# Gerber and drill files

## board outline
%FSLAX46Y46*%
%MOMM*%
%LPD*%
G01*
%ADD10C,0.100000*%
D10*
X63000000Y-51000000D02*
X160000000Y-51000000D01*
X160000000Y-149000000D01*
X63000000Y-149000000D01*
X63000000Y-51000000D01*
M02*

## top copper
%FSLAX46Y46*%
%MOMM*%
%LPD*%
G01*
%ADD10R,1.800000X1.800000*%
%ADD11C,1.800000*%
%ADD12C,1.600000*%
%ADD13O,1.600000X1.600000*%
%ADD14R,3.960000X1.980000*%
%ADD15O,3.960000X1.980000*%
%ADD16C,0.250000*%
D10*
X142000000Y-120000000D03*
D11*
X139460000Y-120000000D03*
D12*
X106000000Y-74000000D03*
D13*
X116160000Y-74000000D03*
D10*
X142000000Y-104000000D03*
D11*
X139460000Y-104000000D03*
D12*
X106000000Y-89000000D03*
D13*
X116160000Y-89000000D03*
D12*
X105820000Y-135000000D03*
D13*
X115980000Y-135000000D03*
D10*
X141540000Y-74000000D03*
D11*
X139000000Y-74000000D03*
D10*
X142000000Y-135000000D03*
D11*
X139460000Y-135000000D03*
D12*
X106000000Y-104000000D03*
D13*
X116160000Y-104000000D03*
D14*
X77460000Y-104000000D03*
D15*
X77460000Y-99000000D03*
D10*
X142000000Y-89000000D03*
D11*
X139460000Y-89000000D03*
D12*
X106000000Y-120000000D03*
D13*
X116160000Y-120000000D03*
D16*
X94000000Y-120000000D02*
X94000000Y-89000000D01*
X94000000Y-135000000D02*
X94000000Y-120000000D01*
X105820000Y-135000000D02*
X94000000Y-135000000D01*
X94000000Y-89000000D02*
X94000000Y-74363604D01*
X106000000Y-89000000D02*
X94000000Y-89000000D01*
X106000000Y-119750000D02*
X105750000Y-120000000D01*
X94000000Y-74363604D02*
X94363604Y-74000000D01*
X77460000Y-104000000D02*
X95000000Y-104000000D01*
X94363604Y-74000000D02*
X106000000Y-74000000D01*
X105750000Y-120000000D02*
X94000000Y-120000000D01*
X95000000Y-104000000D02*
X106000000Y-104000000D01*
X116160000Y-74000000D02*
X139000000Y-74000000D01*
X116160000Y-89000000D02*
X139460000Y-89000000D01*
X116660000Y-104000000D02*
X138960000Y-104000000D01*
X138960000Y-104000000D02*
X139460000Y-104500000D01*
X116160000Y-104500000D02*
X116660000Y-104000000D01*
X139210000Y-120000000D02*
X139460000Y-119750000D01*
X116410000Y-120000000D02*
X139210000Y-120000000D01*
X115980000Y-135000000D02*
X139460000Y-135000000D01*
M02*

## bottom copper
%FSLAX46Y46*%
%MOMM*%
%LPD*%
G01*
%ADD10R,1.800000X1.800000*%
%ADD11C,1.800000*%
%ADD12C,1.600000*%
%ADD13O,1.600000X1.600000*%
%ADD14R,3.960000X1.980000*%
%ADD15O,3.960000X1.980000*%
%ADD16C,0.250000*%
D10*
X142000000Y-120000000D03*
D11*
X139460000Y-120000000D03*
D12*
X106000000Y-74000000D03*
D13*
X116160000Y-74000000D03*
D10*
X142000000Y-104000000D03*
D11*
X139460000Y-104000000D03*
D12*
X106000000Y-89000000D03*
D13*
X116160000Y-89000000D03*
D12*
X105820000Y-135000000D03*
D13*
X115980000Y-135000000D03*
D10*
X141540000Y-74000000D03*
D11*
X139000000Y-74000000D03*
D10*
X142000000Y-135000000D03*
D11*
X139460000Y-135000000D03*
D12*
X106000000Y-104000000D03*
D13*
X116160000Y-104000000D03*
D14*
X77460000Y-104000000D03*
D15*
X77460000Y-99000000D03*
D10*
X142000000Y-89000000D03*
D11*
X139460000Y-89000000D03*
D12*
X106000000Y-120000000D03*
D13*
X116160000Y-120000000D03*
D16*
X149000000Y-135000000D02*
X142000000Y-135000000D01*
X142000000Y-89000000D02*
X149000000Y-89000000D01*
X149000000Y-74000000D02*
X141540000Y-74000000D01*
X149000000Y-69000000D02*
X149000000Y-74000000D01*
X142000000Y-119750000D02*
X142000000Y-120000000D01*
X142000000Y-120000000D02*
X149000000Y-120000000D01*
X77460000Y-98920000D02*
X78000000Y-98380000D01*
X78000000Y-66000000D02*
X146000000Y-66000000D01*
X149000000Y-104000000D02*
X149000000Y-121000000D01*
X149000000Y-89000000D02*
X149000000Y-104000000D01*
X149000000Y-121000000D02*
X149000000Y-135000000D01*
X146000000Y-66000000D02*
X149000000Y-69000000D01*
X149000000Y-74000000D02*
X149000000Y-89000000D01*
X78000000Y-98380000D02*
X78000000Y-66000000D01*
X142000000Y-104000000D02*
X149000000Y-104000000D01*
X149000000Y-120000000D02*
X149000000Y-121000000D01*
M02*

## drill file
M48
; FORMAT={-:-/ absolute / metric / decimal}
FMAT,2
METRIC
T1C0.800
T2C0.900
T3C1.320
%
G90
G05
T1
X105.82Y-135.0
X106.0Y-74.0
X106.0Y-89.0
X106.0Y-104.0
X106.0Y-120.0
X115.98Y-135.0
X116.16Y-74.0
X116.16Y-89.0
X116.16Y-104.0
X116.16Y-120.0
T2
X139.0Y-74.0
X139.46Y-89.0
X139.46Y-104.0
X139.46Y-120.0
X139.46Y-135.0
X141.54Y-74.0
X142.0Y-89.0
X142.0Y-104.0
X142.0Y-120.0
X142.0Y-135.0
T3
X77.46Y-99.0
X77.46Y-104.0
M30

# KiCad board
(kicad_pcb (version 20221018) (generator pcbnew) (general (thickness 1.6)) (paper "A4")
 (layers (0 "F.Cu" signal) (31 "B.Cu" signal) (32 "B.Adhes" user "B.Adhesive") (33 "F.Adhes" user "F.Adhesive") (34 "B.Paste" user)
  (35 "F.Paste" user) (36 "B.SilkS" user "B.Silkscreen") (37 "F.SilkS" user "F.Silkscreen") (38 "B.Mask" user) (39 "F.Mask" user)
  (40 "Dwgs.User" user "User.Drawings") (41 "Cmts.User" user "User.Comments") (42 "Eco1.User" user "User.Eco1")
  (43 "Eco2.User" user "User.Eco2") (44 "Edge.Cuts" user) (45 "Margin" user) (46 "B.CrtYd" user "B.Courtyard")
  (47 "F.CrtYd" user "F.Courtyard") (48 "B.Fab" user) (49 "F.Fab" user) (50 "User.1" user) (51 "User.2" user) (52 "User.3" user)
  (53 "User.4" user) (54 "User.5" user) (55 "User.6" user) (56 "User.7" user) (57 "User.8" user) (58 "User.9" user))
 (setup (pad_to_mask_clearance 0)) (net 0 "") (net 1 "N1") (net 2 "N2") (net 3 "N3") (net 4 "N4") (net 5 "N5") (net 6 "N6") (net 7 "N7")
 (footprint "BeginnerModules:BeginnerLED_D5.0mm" (layer "F.Cu") (at 142 120 180)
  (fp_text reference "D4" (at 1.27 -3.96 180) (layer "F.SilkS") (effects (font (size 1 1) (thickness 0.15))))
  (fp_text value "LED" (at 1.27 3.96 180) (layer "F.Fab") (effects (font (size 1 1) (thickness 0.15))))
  (pad "1" thru_hole rect (at 0 0 180) (size 1.8 1.8) (drill 0.9) (layers "*.Cu" "*.Mask") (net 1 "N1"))
  (pad "2" thru_hole circle (at 2.54 0 180) (size 1.8 1.8) (drill 0.9) (layers "*.Cu" "*.Mask") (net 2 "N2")))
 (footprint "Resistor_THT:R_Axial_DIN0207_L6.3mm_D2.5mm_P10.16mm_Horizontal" (layer "F.Cu") (at 106 74)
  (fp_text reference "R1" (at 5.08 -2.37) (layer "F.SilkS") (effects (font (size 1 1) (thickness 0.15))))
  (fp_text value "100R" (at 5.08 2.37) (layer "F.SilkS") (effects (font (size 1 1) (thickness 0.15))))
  (pad "1" thru_hole circle (at 0 0) (size 1.6 1.6) (drill 0.8) (layers "*.Cu" "*.Mask") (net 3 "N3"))
  (pad "2" thru_hole oval (at 10.16 0) (size 1.6 1.6) (drill 0.8) (layers "*.Cu" "*.Mask") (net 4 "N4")))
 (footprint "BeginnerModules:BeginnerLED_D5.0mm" (layer "F.Cu") (at 142 104 180)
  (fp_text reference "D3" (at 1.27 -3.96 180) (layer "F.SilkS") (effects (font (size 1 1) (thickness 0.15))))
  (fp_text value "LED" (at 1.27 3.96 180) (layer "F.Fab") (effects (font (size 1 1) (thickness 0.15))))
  (pad "1" thru_hole rect (at 0 0 180) (size 1.8 1.8) (drill 0.9) (layers "*.Cu" "*.Mask") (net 1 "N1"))
  (pad "2" thru_hole circle (at 2.54 0 180) (size 1.8 1.8) (drill 0.9) (layers "*.Cu" "*.Mask") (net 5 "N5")))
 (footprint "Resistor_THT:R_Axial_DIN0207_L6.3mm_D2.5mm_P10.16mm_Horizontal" (layer "F.Cu") (at 106 89)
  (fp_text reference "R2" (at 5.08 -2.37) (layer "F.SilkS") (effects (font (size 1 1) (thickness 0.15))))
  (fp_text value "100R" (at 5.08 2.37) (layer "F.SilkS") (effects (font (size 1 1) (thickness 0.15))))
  (pad "1" thru_hole circle (at 0 0) (size 1.6 1.6) (drill 0.8) (layers "*.Cu" "*.Mask") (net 3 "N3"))
  (pad "2" thru_hole oval (at 10.16 0) (size 1.6 1.6) (drill 0.8) (layers "*.Cu" "*.Mask") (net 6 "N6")))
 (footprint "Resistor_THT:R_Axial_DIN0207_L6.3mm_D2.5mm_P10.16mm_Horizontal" (layer "F.Cu") (at 105.82 135)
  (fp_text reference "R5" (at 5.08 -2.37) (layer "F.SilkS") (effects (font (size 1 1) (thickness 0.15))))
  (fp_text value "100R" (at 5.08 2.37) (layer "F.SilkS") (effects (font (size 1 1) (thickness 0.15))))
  (pad "1" thru_hole circle (at 0 0) (size 1.6 1.6) (drill 0.8) (layers "*.Cu" "*.Mask") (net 3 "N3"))
  (pad "2" thru_hole oval (at 10.16 0) (size 1.6 1.6) (drill 0.8) (layers "*.Cu" "*.Mask") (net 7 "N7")))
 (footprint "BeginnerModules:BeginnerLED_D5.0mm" (layer "F.Cu") (at 141.54 74 180)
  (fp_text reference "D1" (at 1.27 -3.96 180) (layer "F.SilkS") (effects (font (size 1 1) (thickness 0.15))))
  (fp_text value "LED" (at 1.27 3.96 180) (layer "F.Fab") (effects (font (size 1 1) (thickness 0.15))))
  (pad "1" thru_hole rect (at 0 0 180) (size 1.8 1.8) (drill 0.9) (layers "*.Cu" "*.Mask") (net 1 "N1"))
  (pad "2" thru_hole circle (at 2.54 0 180) (size 1.8 1.8) (drill 0.9) (layers "*.Cu" "*.Mask") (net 4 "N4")))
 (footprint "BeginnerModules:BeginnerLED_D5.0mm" (layer "F.Cu") (at 142 135 180)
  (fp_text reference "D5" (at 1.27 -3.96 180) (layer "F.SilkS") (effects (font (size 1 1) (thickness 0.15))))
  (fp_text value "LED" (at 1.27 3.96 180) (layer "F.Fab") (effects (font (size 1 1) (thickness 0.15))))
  (pad "1" thru_hole rect (at 0 0 180) (size 1.8 1.8) (drill 0.9) (layers "*.Cu" "*.Mask") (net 1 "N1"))
  (pad "2" thru_hole circle (at 2.54 0 180) (size 1.8 1.8) (drill 0.9) (layers "*.Cu" "*.Mask") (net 7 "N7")))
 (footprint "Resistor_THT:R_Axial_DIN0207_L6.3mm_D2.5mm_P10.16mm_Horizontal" (layer "F.Cu") (at 106 104)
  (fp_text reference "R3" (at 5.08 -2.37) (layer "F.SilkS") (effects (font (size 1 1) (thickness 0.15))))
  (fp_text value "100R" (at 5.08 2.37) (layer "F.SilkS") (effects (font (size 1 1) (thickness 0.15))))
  (pad "1" thru_hole circle (at 0 0) (size 1.6 1.6) (drill 0.8) (layers "*.Cu" "*.Mask") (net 3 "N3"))
  (pad "2" thru_hole oval (at 10.16 0) (size 1.6 1.6) (drill 0.8) (layers "*.Cu" "*.Mask") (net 5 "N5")))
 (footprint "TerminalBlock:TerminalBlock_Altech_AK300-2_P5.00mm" (layer "F.Cu") (at 77.46 104 90)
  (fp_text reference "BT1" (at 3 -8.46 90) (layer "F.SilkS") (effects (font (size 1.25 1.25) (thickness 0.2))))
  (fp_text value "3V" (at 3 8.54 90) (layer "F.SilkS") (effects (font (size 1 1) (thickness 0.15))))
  (pad "1" thru_hole rect (at 0 0 90) (size 1.98 3.96) (drill 1.32) (layers "*.Cu" "*.Mask") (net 3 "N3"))
  (pad "2" thru_hole oval (at 5 0 90) (size 1.98 3.96) (drill 1.32) (layers "*.Cu" "*.Mask") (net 1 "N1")))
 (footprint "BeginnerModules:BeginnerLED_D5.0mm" (layer "F.Cu") (at 142 89 180)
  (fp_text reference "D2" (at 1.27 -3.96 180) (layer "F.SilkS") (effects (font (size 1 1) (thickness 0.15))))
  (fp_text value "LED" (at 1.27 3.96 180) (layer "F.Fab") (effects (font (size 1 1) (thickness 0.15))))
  (pad "1" thru_hole rect (at 0 0 180) (size 1.8 1.8) (drill 0.9) (layers "*.Cu" "*.Mask") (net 1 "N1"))
  (pad "2" thru_hole circle (at 2.54 0 180) (size 1.8 1.8) (drill 0.9) (layers "*.Cu" "*.Mask") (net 6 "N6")))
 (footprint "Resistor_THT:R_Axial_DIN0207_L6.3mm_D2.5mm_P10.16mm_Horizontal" (layer "F.Cu") (at 106 120)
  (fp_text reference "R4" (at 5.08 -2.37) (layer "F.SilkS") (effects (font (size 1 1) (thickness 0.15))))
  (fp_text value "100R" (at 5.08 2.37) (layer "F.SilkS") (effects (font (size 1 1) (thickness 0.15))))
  (pad "1" thru_hole circle (at 0 0) (size 1.6 1.6) (drill 0.8) (layers "*.Cu" "*.Mask") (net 3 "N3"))
  (pad "2" thru_hole oval (at 10.16 0) (size 1.6 1.6) (drill 0.8) (layers "*.Cu" "*.Mask") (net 2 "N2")))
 (gr_rect (start 63 51) (end 160 149) (stroke (width 0.1) (type default)) (fill none) (layer "Edge.Cuts"))
 (segment (start 94 120) (end 94 89) (width 0.25) (layer "F.Cu") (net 3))
 (segment (start 94 135) (end 94 120) (width 0.25) (layer "F.Cu") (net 3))
 (segment (start 105.82 135) (end 94 135) (width 0.25) (layer "F.Cu") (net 3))
 (segment (start 94 89) (end 94 74.363604) (width 0.25) (layer "F.Cu") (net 3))
 (segment (start 106 89) (end 94 89) (width 0.25) (layer "F.Cu") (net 3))
 (segment (start 106 119.75) (end 105.75 120) (width 0.25) (layer "F.Cu") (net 3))
 (segment (start 94 74.363604) (end 94.363604 74) (width 0.25) (layer "F.Cu") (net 3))
 (segment (start 77.46 104) (end 95 104) (width 0.25) (layer "F.Cu") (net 3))
 (segment (start 94.363604 74) (end 106 74) (width 0.25) (layer "F.Cu") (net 3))
 (segment (start 105.75 120) (end 94 120) (width 0.25) (layer "F.Cu") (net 3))
 (segment (start 95 104) (end 106 104) (width 0.25) (layer "F.Cu") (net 3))
 (segment (start 149 135) (end 142 135) (width 0.25) (layer "B.Cu") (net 1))
 (segment (start 142 89) (end 149 89) (width 0.25) (layer "B.Cu") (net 1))
 (segment (start 149 74) (end 141.54 74) (width 0.25) (layer "B.Cu") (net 1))
 (segment (start 149 69) (end 149 74) (width 0.25) (layer "B.Cu") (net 1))
 (segment (start 142 119.75) (end 142 120) (width 0.25) (layer "B.Cu") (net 1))
 (segment (start 142 120) (end 149 120) (width 0.25) (layer "B.Cu") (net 1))
 (segment (start 77.46 98.92) (end 78 98.38) (width 0.25) (layer "B.Cu") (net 1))
 (segment (start 78 66) (end 146 66) (width 0.25) (layer "B.Cu") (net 1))
 (segment (start 149 104) (end 149 121) (width 0.25) (layer "B.Cu") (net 1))
 (segment (start 149 89) (end 149 104) (width 0.25) (layer "B.Cu") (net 1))
 (segment (start 149 121) (end 149 135) (width 0.25) (layer "B.Cu") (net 1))
 (segment (start 146 66) (end 149 69) (width 0.25) (layer "B.Cu") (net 1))
 (segment (start 149 74) (end 149 89) (width 0.25) (layer "B.Cu") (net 1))
 (segment (start 78 98.38) (end 78 66) (width 0.25) (layer "B.Cu") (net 1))
 (segment (start 142 104) (end 149 104) (width 0.25) (layer "B.Cu") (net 1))
 (segment (start 149 120) (end 149 121) (width 0.25) (layer "B.Cu") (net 1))
 (segment (start 116.16 74) (end 139 74) (width 0.25) (layer "F.Cu") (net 4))
 (segment (start 116.16 89) (end 139.46 89) (width 0.25) (layer "F.Cu") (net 6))
 (segment (start 116.66 104) (end 138.96 104) (width 0.25) (layer "F.Cu") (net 5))
 (segment (start 138.96 104) (end 139.46 104.5) (width 0.25) (layer "F.Cu") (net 5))
 (segment (start 116.16 104.5) (end 116.66 104) (width 0.25) (layer "F.Cu") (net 5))
 (segment (start 139.21 120) (end 139.46 119.75) (width 0.25) (layer "F.Cu") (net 2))
 (segment (start 116.41 120) (end 139.21 120) (width 0.25) (layer "F.Cu") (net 2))
 (segment (start 115.98 135) (end 139.46 135) (width 0.25) (layer "F.Cu") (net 7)))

